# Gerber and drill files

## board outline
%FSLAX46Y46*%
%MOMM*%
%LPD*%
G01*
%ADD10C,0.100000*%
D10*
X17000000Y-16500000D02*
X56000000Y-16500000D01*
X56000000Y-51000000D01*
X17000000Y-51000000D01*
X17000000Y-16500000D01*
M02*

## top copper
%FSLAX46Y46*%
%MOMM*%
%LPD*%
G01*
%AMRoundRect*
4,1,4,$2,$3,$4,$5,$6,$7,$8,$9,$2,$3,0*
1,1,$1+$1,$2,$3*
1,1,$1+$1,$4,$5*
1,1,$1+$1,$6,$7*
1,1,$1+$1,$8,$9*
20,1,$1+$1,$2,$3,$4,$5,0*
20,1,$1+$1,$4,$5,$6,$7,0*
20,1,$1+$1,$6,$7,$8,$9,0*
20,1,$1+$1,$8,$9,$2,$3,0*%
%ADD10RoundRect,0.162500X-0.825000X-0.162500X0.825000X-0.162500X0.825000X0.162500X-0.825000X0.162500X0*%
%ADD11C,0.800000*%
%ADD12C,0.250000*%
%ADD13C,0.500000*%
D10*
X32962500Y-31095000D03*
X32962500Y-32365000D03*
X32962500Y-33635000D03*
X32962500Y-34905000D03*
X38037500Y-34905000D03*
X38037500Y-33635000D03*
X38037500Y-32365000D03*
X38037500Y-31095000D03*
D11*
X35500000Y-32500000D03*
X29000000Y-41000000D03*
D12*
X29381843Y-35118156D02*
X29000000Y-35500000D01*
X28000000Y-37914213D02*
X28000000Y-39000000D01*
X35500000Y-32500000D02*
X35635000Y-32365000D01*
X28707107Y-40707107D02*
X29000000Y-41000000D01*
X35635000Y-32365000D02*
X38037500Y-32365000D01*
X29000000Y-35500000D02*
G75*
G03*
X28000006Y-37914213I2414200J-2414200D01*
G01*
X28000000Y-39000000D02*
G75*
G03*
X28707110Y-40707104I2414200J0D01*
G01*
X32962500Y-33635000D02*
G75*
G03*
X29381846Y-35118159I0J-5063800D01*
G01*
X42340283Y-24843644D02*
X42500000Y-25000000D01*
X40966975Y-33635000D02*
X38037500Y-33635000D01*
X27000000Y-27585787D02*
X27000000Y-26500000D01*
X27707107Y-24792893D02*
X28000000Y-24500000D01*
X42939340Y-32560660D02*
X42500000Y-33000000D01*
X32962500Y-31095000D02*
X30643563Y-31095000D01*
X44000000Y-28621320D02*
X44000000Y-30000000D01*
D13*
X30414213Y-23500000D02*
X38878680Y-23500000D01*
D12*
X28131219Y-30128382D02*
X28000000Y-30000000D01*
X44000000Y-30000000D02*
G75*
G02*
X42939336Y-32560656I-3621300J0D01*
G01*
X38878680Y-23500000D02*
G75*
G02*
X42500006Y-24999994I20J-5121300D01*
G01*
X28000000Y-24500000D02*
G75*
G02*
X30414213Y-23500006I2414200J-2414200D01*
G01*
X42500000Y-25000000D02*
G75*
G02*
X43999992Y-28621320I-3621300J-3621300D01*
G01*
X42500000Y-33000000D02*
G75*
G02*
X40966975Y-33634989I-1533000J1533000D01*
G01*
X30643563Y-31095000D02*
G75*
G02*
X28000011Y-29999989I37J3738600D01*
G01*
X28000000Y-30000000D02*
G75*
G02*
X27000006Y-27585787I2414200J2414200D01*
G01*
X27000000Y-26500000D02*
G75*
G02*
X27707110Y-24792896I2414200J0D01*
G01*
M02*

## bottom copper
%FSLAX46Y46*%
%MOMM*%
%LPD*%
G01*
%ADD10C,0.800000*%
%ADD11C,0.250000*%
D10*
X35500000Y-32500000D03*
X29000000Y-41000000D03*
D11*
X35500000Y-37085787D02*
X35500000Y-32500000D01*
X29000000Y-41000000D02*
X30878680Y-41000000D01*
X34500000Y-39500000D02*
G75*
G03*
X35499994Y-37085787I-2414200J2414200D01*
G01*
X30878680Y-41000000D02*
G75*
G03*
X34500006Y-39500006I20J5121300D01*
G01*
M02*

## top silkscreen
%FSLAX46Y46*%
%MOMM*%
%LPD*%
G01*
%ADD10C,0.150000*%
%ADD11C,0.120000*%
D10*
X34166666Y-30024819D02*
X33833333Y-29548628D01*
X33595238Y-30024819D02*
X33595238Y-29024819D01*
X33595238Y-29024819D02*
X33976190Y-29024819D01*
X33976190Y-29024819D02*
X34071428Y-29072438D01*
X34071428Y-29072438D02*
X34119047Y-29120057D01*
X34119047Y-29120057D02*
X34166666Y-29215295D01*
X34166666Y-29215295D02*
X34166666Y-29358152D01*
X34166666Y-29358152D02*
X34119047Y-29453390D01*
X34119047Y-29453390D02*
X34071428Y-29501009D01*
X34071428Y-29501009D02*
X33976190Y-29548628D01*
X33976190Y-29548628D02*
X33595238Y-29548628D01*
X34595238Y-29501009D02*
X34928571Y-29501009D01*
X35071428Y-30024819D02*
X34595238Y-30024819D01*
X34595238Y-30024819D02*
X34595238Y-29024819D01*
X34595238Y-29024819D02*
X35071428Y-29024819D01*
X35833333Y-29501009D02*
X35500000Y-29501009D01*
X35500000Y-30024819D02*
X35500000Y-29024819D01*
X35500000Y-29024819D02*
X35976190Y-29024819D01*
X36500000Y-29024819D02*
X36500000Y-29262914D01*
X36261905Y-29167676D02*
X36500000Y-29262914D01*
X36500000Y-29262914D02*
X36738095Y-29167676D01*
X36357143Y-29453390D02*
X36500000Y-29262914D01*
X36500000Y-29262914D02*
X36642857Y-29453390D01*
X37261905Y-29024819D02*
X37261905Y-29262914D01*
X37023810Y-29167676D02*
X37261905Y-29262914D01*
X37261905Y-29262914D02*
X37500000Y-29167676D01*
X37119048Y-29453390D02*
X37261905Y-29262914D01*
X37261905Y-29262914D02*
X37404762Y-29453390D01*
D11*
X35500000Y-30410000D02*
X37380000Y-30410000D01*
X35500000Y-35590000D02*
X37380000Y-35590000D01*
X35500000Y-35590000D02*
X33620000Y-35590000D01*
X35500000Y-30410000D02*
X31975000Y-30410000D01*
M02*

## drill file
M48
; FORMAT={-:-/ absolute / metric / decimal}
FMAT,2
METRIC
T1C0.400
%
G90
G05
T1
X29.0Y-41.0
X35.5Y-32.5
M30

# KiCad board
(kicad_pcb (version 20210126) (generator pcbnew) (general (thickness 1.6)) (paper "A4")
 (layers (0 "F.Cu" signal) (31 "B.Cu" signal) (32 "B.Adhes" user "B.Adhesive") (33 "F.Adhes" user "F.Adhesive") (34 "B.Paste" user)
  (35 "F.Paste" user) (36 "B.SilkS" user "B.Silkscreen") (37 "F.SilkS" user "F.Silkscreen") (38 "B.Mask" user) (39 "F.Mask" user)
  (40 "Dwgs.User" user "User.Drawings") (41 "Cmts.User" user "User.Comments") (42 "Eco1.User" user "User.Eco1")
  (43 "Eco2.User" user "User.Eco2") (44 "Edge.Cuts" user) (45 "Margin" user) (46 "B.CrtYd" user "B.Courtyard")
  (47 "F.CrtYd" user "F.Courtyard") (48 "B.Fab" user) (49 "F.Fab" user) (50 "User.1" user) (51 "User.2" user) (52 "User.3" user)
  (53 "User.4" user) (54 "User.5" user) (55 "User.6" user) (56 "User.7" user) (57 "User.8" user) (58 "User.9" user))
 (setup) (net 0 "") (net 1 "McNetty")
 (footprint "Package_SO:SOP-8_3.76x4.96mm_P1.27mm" (layer "F.Cu") (at 35.5 33)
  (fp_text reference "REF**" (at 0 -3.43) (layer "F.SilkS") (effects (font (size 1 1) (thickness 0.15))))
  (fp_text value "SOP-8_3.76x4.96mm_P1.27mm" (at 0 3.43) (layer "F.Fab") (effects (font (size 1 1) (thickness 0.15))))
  (fp_line (start 0 -2.59) (end 1.88 -2.59) (layer "F.SilkS") (width 0.12))
  (fp_line (start 0 2.59) (end 1.88 2.59) (layer "F.SilkS") (width 0.12))
  (fp_line (start 0 2.59) (end -1.88 2.59) (layer "F.SilkS") (width 0.12))
  (fp_line (start 0 -2.59) (end -3.525 -2.59) (layer "F.SilkS") (width 0.12))
  (pad "1" smd roundrect (at -2.5375 -1.905) (locked) (size 1.975 0.65) (layers "F.Cu" "F.Paste" "F.Mask") (roundrect_rratio 0.25)
   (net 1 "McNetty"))
  (pad "2" smd roundrect (at -2.5375 -0.635) (locked) (size 1.975 0.65) (layers "F.Cu" "F.Paste" "F.Mask") (roundrect_rratio 0.25))
  (pad "3" smd roundrect (at -2.5375 0.635) (locked) (size 1.975 0.65) (layers "F.Cu" "F.Paste" "F.Mask") (roundrect_rratio 0.25))
  (pad "4" smd roundrect (at -2.5375 1.905) (locked) (size 1.975 0.65) (layers "F.Cu" "F.Paste" "F.Mask") (roundrect_rratio 0.25))
  (pad "5" smd roundrect (at 2.5375 1.905) (locked) (size 1.975 0.65) (layers "F.Cu" "F.Paste" "F.Mask") (roundrect_rratio 0.25))
  (pad "6" smd roundrect (at 2.5375 0.635) (locked) (size 1.975 0.65) (layers "F.Cu" "F.Paste" "F.Mask") (roundrect_rratio 0.25)
   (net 1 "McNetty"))
  (pad "7" smd roundrect (at 2.5375 -0.635) (locked) (size 1.975 0.65) (layers "F.Cu" "F.Paste" "F.Mask") (roundrect_rratio 0.25))
  (pad "8" smd roundrect (at 2.5375 -1.905) (locked) (size 1.975 0.65) (layers "F.Cu" "F.Paste" "F.Mask") (roundrect_rratio 0.25)))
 (gr_rect (start 17 16.5) (end 56 51) (layer "Edge.Cuts") (width 0.1) (fill none))
 (segment (start 29.381843 35.118156) (end 29 35.5) (width 0.25) (layer "F.Cu") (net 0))
 (segment (start 28 37.914213) (end 28 39) (width 0.25) (layer "F.Cu") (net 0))
 (segment (start 35.5 32.5) (end 35.635 32.365) (width 0.25) (layer "F.Cu") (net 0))
 (segment (start 28.707107 40.707107) (end 29 41) (width 0.25) (layer "F.Cu") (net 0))
 (segment (start 35.635 32.365) (end 38.0375 32.365) (width 0.25) (layer "F.Cu") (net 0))
 (via (at 35.5 32.5) (size 0.8) (drill 0.4) (layers "F.Cu" "B.Cu") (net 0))
 (via (at 29 41) (size 0.8) (drill 0.4) (layers "F.Cu" "B.Cu") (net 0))
 (arc (start 29 35.5) (mid 28.259892 36.60765) (end 28 37.914213) (width 0.25) (layer "F.Cu") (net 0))
 (arc (start 28 39) (mid 28.183771 39.92388) (end 28.707107 40.707107) (width 0.25) (layer "F.Cu") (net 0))
 (arc (start 32.9625 33.635) (mid 31.024663 34.02046) (end 29.381843 35.118156) (width 0.25) (layer "F.Cu") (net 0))
 (segment (start 35.5 37.085787) (end 35.5 32.5) (width 0.25) (layer "B.Cu") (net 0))
 (segment (start 29 41) (end 30.87868 41) (width 0.25) (layer "B.Cu") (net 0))
 (arc (start 34.5 39.5) (mid 35.240108 38.39235) (end 35.5 37.085787) (width 0.25) (layer "B.Cu") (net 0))
 (arc (start 30.87868 41) (mid 32.838524 40.610163) (end 34.5 39.5) (width 0.25) (layer "B.Cu") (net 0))
 (segment (start 42.340283 24.843644) (end 42.5 25) (width 0.25) (layer "F.Cu") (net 1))
 (segment (start 40.966975 33.635) (end 38.0375 33.635) (width 0.25) (layer "F.Cu") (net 1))
 (segment (start 27 27.585787) (end 27 26.5) (width 0.25) (layer "F.Cu") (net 1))
 (segment (start 27.707107 24.792893) (end 28 24.5) (width 0.25) (layer "F.Cu") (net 1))
 (segment (start 42.93934 32.56066) (end 42.5 33) (width 0.25) (layer "F.Cu") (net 1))
 (segment (start 32.9625 31.095) (end 30.643563 31.095) (width 0.25) (layer "F.Cu") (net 1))
 (segment (start 44 28.62132) (end 44 30) (width 0.25) (layer "F.Cu") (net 1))
 (segment (start 30.414213 23.5) (end 38.87868 23.5) (width 0.5) (layer "F.Cu") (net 1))
 (segment (start 28.131219 30.128382) (end 28 30) (width 0.25) (layer "F.Cu") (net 1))
 (arc (start 44 30) (mid 43.724343 31.385819) (end 42.93934 32.56066) (width 0.25) (layer "F.Cu") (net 1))
 (arc (start 38.87868 23.5) (mid 40.838524 23.889837) (end 42.5 25) (width 0.25) (layer "F.Cu") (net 1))
 (arc (start 28 24.5) (mid 29.10765 23.759892) (end 30.414213 23.5) (width 0.25) (layer "F.Cu") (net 1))
 (arc (start 42.5 25) (mid 43.610163 26.661476) (end 44 28.62132) (width 0.25) (layer "F.Cu") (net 1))
 (arc (start 42.5 33) (mid 41.796643 33.469969) (end 40.966975 33.635) (width 0.25) (layer "F.Cu") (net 1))
 (arc (start 30.643563 31.095) (mid 29.212877 30.810419) (end 28 30) (width 0.25) (layer "F.Cu") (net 1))
 (arc (start 28 30) (mid 27.259892 28.89235) (end 27 27.585787) (width 0.25) (layer "F.Cu") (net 1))
 (arc (start 27 26.5) (mid 27.183771 25.57612) (end 27.707107 24.792893) (width 0.25) (layer "F.Cu") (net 1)))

